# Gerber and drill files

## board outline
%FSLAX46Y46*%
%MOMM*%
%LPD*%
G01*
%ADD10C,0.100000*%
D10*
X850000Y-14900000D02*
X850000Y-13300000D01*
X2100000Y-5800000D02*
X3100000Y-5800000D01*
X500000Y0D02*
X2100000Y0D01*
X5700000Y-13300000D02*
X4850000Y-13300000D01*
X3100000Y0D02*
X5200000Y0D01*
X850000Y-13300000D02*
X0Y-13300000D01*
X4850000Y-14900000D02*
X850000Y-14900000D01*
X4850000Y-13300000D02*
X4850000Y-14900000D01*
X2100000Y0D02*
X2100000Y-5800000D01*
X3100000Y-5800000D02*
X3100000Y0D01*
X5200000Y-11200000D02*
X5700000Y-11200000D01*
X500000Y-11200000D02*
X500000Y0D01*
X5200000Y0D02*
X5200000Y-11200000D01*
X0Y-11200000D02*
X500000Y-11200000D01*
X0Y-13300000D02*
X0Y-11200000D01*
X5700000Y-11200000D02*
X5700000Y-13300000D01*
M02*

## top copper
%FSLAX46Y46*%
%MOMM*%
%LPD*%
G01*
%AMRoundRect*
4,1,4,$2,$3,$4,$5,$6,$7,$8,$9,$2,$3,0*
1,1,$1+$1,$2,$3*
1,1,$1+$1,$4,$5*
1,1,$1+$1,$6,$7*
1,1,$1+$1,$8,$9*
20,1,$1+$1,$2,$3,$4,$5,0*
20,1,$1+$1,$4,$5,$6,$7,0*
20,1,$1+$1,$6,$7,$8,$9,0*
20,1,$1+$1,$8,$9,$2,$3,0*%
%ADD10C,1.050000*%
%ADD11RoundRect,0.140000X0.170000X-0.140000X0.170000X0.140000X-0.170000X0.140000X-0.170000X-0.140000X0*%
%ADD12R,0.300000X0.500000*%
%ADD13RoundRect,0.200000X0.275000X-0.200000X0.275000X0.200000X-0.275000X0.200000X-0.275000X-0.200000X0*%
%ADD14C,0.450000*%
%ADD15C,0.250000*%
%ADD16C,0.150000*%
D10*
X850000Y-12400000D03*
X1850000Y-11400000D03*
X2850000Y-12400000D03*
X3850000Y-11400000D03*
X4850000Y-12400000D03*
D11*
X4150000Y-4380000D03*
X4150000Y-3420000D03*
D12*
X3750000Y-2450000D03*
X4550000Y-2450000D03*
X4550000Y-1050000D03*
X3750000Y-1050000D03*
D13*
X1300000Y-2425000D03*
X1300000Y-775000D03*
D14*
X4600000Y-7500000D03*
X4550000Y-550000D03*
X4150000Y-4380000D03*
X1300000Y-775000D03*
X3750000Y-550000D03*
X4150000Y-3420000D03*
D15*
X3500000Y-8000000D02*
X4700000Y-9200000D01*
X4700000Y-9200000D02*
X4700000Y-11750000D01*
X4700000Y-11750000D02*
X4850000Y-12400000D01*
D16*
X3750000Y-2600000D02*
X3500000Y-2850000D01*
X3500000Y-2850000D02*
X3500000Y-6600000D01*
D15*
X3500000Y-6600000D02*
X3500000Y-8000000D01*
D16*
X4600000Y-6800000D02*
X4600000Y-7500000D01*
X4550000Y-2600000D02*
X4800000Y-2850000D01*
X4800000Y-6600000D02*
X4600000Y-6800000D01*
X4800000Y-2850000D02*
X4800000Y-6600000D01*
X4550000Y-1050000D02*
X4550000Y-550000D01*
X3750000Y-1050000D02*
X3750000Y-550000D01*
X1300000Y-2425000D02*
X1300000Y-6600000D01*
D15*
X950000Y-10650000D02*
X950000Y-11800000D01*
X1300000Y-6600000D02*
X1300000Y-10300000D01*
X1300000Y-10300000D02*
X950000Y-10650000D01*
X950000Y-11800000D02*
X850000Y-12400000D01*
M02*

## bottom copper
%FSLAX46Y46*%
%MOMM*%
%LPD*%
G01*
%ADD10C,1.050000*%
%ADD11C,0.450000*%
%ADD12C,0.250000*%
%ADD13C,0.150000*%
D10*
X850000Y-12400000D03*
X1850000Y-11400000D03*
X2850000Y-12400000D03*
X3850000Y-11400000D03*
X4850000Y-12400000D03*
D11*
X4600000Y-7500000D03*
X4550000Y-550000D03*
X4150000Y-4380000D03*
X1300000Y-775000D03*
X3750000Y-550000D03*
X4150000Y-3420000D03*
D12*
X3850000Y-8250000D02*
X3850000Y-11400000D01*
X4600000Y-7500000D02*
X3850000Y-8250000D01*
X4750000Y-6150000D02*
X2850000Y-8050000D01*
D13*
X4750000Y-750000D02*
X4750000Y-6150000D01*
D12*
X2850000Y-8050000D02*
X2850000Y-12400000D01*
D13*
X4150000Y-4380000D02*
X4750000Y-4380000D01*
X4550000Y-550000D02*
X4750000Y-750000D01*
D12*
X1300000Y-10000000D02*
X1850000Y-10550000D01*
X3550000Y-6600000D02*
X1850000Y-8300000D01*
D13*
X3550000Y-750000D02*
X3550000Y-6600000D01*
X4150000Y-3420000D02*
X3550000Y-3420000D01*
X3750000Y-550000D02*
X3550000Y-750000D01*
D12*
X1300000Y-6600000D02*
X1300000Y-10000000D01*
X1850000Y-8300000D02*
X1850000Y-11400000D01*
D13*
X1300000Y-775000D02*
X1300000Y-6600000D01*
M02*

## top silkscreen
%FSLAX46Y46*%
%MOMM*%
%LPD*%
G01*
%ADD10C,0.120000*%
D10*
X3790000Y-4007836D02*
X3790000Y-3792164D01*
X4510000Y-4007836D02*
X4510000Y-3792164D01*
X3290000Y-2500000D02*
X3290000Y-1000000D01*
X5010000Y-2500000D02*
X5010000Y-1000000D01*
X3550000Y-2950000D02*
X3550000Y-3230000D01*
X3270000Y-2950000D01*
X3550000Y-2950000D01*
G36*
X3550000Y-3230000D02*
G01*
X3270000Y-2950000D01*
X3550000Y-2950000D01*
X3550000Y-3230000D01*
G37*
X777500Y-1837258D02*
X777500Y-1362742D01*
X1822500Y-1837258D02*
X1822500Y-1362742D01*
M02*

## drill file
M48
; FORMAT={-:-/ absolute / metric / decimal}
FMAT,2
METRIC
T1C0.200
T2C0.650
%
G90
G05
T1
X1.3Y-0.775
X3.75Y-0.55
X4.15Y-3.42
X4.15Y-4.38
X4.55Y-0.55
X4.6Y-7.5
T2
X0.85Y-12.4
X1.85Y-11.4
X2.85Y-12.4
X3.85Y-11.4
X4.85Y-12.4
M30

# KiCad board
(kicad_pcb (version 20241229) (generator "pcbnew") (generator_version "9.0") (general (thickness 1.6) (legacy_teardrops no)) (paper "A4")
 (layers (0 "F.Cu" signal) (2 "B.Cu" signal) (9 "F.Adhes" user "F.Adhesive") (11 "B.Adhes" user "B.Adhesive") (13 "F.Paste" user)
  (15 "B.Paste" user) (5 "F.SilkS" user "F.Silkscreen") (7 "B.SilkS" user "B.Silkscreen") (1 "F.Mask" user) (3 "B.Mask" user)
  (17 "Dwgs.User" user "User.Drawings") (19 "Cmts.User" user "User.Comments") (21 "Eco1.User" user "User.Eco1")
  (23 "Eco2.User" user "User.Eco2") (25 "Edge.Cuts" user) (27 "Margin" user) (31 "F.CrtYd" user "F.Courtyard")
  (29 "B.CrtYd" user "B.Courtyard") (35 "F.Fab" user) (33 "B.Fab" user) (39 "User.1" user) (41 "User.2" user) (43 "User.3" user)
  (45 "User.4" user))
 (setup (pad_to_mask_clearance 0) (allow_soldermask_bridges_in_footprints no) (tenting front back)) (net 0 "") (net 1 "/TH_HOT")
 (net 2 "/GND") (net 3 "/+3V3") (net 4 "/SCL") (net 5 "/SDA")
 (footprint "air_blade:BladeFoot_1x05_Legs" (layer "F.Cu") (at 2.85 12.4)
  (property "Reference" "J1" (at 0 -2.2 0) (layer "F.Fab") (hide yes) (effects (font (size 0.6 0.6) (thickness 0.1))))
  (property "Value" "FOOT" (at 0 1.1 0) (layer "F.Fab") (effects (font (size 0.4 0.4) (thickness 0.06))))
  (pad "1" thru_hole circle (at -2 0) (size 1.05 1.05) (drill 0.65) (layers "*.Cu" "*.Mask") (remove_unused_layers no) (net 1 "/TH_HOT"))
  (pad "2" thru_hole circle (at -1 -1) (size 1.05 1.05) (drill 0.65) (layers "*.Cu" "*.Mask") (remove_unused_layers no) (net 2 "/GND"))
  (pad "3" thru_hole circle (at 0 0) (size 1.05 1.05) (drill 0.65) (layers "*.Cu" "*.Mask") (remove_unused_layers no) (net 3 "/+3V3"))
  (pad "4" thru_hole circle (at 1 -1) (size 1.05 1.05) (drill 0.65) (layers "*.Cu" "*.Mask") (remove_unused_layers no) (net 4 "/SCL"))
  (pad "5" thru_hole circle (at 2 0) (size 1.05 1.05) (drill 0.65) (layers "*.Cu" "*.Mask") (remove_unused_layers no) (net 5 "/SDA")))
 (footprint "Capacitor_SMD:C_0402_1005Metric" (layer "F.Cu") (at 4.15 3.9 90)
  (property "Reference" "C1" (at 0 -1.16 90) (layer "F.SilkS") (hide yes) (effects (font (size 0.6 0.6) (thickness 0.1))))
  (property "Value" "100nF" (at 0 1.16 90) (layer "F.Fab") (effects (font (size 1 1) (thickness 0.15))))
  (fp_line (start -0.107836 -0.36) (end 0.107836 -0.36) (stroke (width 0.12) (type solid)) (layer "F.SilkS"))
  (fp_line (start -0.107836 0.36) (end 0.107836 0.36) (stroke (width 0.12) (type solid)) (layer "F.SilkS"))
  (pad "1" smd roundrect (at -0.48 0 90) (size 0.56 0.62) (layers "F.Cu" "F.Mask" "F.Paste") (roundrect_rratio 0.25) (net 3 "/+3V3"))
  (pad "2" smd roundrect (at 0.48 0 90) (size 0.56 0.62) (layers "F.Cu" "F.Mask" "F.Paste") (roundrect_rratio 0.25) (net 2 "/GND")))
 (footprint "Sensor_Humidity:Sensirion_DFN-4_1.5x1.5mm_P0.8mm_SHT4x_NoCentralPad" (layer "F.Cu") (at 4.15 1.75 90)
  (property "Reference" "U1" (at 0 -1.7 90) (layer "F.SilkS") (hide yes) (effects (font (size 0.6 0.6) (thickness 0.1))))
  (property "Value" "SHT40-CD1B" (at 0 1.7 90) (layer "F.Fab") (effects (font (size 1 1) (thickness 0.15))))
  (fp_line (start -0.75 -0.86) (end 0.75 -0.86) (stroke (width 0.12) (type solid)) (layer "F.SilkS"))
  (fp_line (start -0.75 0.86) (end 0.75 0.86) (stroke (width 0.12) (type solid)) (layer "F.SilkS"))
  (fp_poly
   (pts (xy -1.2 -0.6) (xy -1.48 -0.6) (xy -1.2 -0.88) (xy -1.2 -0.6)) (stroke (width 0.12) (type solid)) (fill yes) (layer "F.SilkS"))
  (pad "1" smd rect (at -0.7 -0.4 90) (size 0.5 0.3) (layers "F.Cu" "F.Mask" "F.Paste") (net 5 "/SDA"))
  (pad "2" smd rect (at -0.7 0.4 90) (size 0.5 0.3) (layers "F.Cu" "F.Mask" "F.Paste") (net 4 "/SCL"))
  (pad "3" smd rect (at 0.7 0.4 90) (size 0.5 0.3) (layers "F.Cu" "F.Mask" "F.Paste") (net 3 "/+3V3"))
  (pad "4" smd rect (at 0.7 -0.4 90) (size 0.5 0.3) (layers "F.Cu" "F.Mask" "F.Paste") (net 2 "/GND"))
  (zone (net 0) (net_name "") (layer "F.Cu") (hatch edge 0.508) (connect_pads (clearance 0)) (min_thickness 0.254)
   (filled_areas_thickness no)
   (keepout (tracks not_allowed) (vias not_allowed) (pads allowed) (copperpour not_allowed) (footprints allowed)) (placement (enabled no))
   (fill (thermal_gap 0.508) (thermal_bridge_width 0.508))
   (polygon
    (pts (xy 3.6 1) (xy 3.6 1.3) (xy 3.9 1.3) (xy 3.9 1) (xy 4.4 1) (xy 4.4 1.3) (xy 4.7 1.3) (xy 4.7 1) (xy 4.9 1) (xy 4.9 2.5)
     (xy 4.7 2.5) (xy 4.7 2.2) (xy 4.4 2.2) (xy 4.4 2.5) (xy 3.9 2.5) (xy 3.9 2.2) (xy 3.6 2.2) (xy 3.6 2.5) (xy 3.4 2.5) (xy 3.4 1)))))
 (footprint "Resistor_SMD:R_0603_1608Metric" (layer "F.Cu") (at 1.3 1.6 90)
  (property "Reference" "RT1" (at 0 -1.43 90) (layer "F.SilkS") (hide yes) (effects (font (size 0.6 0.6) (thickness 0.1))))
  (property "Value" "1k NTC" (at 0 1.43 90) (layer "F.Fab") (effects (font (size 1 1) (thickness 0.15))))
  (fp_line (start -0.237258 -0.5225) (end 0.237258 -0.5225) (stroke (width 0.12) (type solid)) (layer "F.SilkS"))
  (fp_line (start -0.237258 0.5225) (end 0.237258 0.5225) (stroke (width 0.12) (type solid)) (layer "F.SilkS"))
  (pad "1" smd roundrect (at -0.825 0 90) (size 0.8 0.95) (layers "F.Cu" "F.Mask" "F.Paste") (roundrect_rratio 0.25) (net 1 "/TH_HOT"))
  (pad "2" smd roundrect (at 0.825 0 90) (size 0.8 0.95) (layers "F.Cu" "F.Mask" "F.Paste") (roundrect_rratio 0.25) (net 2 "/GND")))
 (gr_line (start 0.85 14.9) (end 0.85 13.3) (stroke (width 0.1) (type default)) (layer "Edge.Cuts"))
 (gr_line (start 2.1 5.8) (end 3.1 5.8) (stroke (width 0.1) (type default)) (layer "Edge.Cuts"))
 (gr_line (start 0.5 0) (end 2.1 0) (stroke (width 0.1) (type default)) (layer "Edge.Cuts"))
 (gr_line (start 5.7 13.3) (end 4.85 13.3) (stroke (width 0.1) (type default)) (layer "Edge.Cuts"))
 (gr_line (start 3.1 0) (end 5.2 0) (stroke (width 0.1) (type default)) (layer "Edge.Cuts"))
 (gr_line (start 0.85 13.3) (end 0 13.3) (stroke (width 0.1) (type default)) (layer "Edge.Cuts"))
 (gr_line (start 4.85 14.9) (end 0.85 14.9) (stroke (width 0.1) (type default)) (layer "Edge.Cuts"))
 (gr_line (start 4.85 13.3) (end 4.85 14.9) (stroke (width 0.1) (type default)) (layer "Edge.Cuts"))
 (gr_line (start 2.1 0) (end 2.1 5.8) (stroke (width 0.1) (type default)) (layer "Edge.Cuts"))
 (gr_line (start 3.1 5.8) (end 3.1 0) (stroke (width 0.1) (type default)) (layer "Edge.Cuts"))
 (gr_line (start 5.2 11.2) (end 5.7 11.2) (stroke (width 0.1) (type default)) (layer "Edge.Cuts"))
 (gr_line (start 0.5 11.2) (end 0.5 0) (stroke (width 0.1) (type default)) (layer "Edge.Cuts"))
 (gr_line (start 5.2 0) (end 5.2 11.2) (stroke (width 0.1) (type default)) (layer "Edge.Cuts"))
 (gr_line (start 0 11.2) (end 0.5 11.2) (stroke (width 0.1) (type default)) (layer "Edge.Cuts"))
 (gr_line (start 0 13.3) (end 0 11.2) (stroke (width 0.1) (type default)) (layer "Edge.Cuts"))
 (gr_line (start 5.7 11.2) (end 5.7 13.3) (stroke (width 0.1) (type default)) (layer "Edge.Cuts"))
 (segment (start 3.5 8) (end 4.7 9.2) (width 0.25) (locked yes) (layer "F.Cu") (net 5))
 (segment (start 4.7 9.2) (end 4.7 11.75) (width 0.25) (locked yes) (layer "F.Cu") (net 5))
 (segment (start 4.7 11.75) (end 4.85 12.4) (width 0.25) (locked yes) (layer "F.Cu") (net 5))
 (segment (start 3.75 2.6) (end 3.5 2.85) (width 0.15) (locked yes) (layer "F.Cu") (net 5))
 (segment (start 3.5 2.85) (end 3.5 6.6) (width 0.15) (locked yes) (layer "F.Cu") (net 5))
 (segment (start 3.5 6.6) (end 3.5 8) (width 0.25) (locked yes) (layer "F.Cu") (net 5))
 (segment (start 4.6 6.8) (end 4.6 7.5) (width 0.15) (locked yes) (layer "F.Cu") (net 4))
 (segment (start 4.55 2.6) (end 4.8 2.85) (width 0.15) (locked yes) (layer "F.Cu") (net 4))
 (segment (start 4.8 6.6) (end 4.6 6.8) (width 0.15) (locked yes) (layer "F.Cu") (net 4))
 (segment (start 4.8 2.85) (end 4.8 6.6) (width 0.15) (locked yes) (layer "F.Cu") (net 4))
 (via (at 4.6 7.5) (size 0.45) (drill 0.2) (layers "F.Cu" "B.Cu") (locked yes) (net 4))
 (segment (start 3.85 8.25) (end 3.85 11.4) (width 0.25) (locked yes) (layer "B.Cu") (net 4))
 (segment (start 4.6 7.5) (end 3.85 8.25) (width 0.25) (locked yes) (layer "B.Cu") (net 4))
 (segment (start 4.55 1.05) (end 4.55 0.55) (width 0.15) (locked yes) (layer "F.Cu") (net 3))
 (via (at 4.55 0.55) (size 0.45) (drill 0.2) (layers "F.Cu" "B.Cu") (locked yes) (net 3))
 (via (at 4.15 4.38) (size 0.45) (drill 0.2) (layers "F.Cu" "B.Cu") (locked yes) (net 3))
 (segment (start 4.75 6.15) (end 2.85 8.05) (width 0.25) (locked yes) (layer "B.Cu") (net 3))
 (segment (start 4.75 0.75) (end 4.75 6.15) (width 0.15) (locked yes) (layer "B.Cu") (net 3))
 (segment (start 2.85 8.05) (end 2.85 12.4) (width 0.25) (locked yes) (layer "B.Cu") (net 3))
 (segment (start 4.15 4.38) (end 4.75 4.38) (width 0.15) (locked yes) (layer "B.Cu") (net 3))
 (segment (start 4.55 0.55) (end 4.75 0.75) (width 0.15) (locked yes) (layer "B.Cu") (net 3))
 (segment (start 3.75 1.05) (end 3.75 0.55) (width 0.15) (locked yes) (layer "F.Cu") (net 2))
 (via (at 1.3 0.775) (size 0.45) (drill 0.2) (layers "F.Cu" "B.Cu") (locked yes) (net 2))
 (via (at 3.75 0.55) (size 0.45) (drill 0.2) (layers "F.Cu" "B.Cu") (locked yes) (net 2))
 (via (at 4.15 3.42) (size 0.45) (drill 0.2) (layers "F.Cu" "B.Cu") (locked yes) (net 2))
 (segment (start 1.3 10) (end 1.85 10.55) (width 0.25) (locked yes) (layer "B.Cu") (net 2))
 (segment (start 3.55 6.6) (end 1.85 8.3) (width 0.25) (locked yes) (layer "B.Cu") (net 2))
 (segment (start 3.55 0.75) (end 3.55 6.6) (width 0.15) (locked yes) (layer "B.Cu") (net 2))
 (segment (start 4.15 3.42) (end 3.55 3.42) (width 0.15) (locked yes) (layer "B.Cu") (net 2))
 (segment (start 3.75 0.55) (end 3.55 0.75) (width 0.15) (locked yes) (layer "B.Cu") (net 2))
 (segment (start 1.3 6.6) (end 1.3 10) (width 0.25) (locked yes) (layer "B.Cu") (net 2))
 (segment (start 1.85 8.3) (end 1.85 11.4) (width 0.25) (locked yes) (layer "B.Cu") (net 2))
 (segment (start 1.3 0.775) (end 1.3 6.6) (width 0.15) (locked yes) (layer "B.Cu") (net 2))
 (segment (start 1.3 2.425) (end 1.3 6.6) (width 0.15) (locked yes) (layer "F.Cu") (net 1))
 (segment (start 0.95 10.65) (end 0.95 11.8) (width 0.25) (locked yes) (layer "F.Cu") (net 1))
 (segment (start 1.3 6.6) (end 1.3 10.3) (width 0.25) (locked yes) (layer "F.Cu") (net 1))
 (segment (start 1.3 10.3) (end 0.95 10.65) (width 0.25) (locked yes) (layer "F.Cu") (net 1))
 (segment (start 0.95 11.8) (end 0.85 12.4) (width 0.25) (locked yes) (layer "F.Cu") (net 1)))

